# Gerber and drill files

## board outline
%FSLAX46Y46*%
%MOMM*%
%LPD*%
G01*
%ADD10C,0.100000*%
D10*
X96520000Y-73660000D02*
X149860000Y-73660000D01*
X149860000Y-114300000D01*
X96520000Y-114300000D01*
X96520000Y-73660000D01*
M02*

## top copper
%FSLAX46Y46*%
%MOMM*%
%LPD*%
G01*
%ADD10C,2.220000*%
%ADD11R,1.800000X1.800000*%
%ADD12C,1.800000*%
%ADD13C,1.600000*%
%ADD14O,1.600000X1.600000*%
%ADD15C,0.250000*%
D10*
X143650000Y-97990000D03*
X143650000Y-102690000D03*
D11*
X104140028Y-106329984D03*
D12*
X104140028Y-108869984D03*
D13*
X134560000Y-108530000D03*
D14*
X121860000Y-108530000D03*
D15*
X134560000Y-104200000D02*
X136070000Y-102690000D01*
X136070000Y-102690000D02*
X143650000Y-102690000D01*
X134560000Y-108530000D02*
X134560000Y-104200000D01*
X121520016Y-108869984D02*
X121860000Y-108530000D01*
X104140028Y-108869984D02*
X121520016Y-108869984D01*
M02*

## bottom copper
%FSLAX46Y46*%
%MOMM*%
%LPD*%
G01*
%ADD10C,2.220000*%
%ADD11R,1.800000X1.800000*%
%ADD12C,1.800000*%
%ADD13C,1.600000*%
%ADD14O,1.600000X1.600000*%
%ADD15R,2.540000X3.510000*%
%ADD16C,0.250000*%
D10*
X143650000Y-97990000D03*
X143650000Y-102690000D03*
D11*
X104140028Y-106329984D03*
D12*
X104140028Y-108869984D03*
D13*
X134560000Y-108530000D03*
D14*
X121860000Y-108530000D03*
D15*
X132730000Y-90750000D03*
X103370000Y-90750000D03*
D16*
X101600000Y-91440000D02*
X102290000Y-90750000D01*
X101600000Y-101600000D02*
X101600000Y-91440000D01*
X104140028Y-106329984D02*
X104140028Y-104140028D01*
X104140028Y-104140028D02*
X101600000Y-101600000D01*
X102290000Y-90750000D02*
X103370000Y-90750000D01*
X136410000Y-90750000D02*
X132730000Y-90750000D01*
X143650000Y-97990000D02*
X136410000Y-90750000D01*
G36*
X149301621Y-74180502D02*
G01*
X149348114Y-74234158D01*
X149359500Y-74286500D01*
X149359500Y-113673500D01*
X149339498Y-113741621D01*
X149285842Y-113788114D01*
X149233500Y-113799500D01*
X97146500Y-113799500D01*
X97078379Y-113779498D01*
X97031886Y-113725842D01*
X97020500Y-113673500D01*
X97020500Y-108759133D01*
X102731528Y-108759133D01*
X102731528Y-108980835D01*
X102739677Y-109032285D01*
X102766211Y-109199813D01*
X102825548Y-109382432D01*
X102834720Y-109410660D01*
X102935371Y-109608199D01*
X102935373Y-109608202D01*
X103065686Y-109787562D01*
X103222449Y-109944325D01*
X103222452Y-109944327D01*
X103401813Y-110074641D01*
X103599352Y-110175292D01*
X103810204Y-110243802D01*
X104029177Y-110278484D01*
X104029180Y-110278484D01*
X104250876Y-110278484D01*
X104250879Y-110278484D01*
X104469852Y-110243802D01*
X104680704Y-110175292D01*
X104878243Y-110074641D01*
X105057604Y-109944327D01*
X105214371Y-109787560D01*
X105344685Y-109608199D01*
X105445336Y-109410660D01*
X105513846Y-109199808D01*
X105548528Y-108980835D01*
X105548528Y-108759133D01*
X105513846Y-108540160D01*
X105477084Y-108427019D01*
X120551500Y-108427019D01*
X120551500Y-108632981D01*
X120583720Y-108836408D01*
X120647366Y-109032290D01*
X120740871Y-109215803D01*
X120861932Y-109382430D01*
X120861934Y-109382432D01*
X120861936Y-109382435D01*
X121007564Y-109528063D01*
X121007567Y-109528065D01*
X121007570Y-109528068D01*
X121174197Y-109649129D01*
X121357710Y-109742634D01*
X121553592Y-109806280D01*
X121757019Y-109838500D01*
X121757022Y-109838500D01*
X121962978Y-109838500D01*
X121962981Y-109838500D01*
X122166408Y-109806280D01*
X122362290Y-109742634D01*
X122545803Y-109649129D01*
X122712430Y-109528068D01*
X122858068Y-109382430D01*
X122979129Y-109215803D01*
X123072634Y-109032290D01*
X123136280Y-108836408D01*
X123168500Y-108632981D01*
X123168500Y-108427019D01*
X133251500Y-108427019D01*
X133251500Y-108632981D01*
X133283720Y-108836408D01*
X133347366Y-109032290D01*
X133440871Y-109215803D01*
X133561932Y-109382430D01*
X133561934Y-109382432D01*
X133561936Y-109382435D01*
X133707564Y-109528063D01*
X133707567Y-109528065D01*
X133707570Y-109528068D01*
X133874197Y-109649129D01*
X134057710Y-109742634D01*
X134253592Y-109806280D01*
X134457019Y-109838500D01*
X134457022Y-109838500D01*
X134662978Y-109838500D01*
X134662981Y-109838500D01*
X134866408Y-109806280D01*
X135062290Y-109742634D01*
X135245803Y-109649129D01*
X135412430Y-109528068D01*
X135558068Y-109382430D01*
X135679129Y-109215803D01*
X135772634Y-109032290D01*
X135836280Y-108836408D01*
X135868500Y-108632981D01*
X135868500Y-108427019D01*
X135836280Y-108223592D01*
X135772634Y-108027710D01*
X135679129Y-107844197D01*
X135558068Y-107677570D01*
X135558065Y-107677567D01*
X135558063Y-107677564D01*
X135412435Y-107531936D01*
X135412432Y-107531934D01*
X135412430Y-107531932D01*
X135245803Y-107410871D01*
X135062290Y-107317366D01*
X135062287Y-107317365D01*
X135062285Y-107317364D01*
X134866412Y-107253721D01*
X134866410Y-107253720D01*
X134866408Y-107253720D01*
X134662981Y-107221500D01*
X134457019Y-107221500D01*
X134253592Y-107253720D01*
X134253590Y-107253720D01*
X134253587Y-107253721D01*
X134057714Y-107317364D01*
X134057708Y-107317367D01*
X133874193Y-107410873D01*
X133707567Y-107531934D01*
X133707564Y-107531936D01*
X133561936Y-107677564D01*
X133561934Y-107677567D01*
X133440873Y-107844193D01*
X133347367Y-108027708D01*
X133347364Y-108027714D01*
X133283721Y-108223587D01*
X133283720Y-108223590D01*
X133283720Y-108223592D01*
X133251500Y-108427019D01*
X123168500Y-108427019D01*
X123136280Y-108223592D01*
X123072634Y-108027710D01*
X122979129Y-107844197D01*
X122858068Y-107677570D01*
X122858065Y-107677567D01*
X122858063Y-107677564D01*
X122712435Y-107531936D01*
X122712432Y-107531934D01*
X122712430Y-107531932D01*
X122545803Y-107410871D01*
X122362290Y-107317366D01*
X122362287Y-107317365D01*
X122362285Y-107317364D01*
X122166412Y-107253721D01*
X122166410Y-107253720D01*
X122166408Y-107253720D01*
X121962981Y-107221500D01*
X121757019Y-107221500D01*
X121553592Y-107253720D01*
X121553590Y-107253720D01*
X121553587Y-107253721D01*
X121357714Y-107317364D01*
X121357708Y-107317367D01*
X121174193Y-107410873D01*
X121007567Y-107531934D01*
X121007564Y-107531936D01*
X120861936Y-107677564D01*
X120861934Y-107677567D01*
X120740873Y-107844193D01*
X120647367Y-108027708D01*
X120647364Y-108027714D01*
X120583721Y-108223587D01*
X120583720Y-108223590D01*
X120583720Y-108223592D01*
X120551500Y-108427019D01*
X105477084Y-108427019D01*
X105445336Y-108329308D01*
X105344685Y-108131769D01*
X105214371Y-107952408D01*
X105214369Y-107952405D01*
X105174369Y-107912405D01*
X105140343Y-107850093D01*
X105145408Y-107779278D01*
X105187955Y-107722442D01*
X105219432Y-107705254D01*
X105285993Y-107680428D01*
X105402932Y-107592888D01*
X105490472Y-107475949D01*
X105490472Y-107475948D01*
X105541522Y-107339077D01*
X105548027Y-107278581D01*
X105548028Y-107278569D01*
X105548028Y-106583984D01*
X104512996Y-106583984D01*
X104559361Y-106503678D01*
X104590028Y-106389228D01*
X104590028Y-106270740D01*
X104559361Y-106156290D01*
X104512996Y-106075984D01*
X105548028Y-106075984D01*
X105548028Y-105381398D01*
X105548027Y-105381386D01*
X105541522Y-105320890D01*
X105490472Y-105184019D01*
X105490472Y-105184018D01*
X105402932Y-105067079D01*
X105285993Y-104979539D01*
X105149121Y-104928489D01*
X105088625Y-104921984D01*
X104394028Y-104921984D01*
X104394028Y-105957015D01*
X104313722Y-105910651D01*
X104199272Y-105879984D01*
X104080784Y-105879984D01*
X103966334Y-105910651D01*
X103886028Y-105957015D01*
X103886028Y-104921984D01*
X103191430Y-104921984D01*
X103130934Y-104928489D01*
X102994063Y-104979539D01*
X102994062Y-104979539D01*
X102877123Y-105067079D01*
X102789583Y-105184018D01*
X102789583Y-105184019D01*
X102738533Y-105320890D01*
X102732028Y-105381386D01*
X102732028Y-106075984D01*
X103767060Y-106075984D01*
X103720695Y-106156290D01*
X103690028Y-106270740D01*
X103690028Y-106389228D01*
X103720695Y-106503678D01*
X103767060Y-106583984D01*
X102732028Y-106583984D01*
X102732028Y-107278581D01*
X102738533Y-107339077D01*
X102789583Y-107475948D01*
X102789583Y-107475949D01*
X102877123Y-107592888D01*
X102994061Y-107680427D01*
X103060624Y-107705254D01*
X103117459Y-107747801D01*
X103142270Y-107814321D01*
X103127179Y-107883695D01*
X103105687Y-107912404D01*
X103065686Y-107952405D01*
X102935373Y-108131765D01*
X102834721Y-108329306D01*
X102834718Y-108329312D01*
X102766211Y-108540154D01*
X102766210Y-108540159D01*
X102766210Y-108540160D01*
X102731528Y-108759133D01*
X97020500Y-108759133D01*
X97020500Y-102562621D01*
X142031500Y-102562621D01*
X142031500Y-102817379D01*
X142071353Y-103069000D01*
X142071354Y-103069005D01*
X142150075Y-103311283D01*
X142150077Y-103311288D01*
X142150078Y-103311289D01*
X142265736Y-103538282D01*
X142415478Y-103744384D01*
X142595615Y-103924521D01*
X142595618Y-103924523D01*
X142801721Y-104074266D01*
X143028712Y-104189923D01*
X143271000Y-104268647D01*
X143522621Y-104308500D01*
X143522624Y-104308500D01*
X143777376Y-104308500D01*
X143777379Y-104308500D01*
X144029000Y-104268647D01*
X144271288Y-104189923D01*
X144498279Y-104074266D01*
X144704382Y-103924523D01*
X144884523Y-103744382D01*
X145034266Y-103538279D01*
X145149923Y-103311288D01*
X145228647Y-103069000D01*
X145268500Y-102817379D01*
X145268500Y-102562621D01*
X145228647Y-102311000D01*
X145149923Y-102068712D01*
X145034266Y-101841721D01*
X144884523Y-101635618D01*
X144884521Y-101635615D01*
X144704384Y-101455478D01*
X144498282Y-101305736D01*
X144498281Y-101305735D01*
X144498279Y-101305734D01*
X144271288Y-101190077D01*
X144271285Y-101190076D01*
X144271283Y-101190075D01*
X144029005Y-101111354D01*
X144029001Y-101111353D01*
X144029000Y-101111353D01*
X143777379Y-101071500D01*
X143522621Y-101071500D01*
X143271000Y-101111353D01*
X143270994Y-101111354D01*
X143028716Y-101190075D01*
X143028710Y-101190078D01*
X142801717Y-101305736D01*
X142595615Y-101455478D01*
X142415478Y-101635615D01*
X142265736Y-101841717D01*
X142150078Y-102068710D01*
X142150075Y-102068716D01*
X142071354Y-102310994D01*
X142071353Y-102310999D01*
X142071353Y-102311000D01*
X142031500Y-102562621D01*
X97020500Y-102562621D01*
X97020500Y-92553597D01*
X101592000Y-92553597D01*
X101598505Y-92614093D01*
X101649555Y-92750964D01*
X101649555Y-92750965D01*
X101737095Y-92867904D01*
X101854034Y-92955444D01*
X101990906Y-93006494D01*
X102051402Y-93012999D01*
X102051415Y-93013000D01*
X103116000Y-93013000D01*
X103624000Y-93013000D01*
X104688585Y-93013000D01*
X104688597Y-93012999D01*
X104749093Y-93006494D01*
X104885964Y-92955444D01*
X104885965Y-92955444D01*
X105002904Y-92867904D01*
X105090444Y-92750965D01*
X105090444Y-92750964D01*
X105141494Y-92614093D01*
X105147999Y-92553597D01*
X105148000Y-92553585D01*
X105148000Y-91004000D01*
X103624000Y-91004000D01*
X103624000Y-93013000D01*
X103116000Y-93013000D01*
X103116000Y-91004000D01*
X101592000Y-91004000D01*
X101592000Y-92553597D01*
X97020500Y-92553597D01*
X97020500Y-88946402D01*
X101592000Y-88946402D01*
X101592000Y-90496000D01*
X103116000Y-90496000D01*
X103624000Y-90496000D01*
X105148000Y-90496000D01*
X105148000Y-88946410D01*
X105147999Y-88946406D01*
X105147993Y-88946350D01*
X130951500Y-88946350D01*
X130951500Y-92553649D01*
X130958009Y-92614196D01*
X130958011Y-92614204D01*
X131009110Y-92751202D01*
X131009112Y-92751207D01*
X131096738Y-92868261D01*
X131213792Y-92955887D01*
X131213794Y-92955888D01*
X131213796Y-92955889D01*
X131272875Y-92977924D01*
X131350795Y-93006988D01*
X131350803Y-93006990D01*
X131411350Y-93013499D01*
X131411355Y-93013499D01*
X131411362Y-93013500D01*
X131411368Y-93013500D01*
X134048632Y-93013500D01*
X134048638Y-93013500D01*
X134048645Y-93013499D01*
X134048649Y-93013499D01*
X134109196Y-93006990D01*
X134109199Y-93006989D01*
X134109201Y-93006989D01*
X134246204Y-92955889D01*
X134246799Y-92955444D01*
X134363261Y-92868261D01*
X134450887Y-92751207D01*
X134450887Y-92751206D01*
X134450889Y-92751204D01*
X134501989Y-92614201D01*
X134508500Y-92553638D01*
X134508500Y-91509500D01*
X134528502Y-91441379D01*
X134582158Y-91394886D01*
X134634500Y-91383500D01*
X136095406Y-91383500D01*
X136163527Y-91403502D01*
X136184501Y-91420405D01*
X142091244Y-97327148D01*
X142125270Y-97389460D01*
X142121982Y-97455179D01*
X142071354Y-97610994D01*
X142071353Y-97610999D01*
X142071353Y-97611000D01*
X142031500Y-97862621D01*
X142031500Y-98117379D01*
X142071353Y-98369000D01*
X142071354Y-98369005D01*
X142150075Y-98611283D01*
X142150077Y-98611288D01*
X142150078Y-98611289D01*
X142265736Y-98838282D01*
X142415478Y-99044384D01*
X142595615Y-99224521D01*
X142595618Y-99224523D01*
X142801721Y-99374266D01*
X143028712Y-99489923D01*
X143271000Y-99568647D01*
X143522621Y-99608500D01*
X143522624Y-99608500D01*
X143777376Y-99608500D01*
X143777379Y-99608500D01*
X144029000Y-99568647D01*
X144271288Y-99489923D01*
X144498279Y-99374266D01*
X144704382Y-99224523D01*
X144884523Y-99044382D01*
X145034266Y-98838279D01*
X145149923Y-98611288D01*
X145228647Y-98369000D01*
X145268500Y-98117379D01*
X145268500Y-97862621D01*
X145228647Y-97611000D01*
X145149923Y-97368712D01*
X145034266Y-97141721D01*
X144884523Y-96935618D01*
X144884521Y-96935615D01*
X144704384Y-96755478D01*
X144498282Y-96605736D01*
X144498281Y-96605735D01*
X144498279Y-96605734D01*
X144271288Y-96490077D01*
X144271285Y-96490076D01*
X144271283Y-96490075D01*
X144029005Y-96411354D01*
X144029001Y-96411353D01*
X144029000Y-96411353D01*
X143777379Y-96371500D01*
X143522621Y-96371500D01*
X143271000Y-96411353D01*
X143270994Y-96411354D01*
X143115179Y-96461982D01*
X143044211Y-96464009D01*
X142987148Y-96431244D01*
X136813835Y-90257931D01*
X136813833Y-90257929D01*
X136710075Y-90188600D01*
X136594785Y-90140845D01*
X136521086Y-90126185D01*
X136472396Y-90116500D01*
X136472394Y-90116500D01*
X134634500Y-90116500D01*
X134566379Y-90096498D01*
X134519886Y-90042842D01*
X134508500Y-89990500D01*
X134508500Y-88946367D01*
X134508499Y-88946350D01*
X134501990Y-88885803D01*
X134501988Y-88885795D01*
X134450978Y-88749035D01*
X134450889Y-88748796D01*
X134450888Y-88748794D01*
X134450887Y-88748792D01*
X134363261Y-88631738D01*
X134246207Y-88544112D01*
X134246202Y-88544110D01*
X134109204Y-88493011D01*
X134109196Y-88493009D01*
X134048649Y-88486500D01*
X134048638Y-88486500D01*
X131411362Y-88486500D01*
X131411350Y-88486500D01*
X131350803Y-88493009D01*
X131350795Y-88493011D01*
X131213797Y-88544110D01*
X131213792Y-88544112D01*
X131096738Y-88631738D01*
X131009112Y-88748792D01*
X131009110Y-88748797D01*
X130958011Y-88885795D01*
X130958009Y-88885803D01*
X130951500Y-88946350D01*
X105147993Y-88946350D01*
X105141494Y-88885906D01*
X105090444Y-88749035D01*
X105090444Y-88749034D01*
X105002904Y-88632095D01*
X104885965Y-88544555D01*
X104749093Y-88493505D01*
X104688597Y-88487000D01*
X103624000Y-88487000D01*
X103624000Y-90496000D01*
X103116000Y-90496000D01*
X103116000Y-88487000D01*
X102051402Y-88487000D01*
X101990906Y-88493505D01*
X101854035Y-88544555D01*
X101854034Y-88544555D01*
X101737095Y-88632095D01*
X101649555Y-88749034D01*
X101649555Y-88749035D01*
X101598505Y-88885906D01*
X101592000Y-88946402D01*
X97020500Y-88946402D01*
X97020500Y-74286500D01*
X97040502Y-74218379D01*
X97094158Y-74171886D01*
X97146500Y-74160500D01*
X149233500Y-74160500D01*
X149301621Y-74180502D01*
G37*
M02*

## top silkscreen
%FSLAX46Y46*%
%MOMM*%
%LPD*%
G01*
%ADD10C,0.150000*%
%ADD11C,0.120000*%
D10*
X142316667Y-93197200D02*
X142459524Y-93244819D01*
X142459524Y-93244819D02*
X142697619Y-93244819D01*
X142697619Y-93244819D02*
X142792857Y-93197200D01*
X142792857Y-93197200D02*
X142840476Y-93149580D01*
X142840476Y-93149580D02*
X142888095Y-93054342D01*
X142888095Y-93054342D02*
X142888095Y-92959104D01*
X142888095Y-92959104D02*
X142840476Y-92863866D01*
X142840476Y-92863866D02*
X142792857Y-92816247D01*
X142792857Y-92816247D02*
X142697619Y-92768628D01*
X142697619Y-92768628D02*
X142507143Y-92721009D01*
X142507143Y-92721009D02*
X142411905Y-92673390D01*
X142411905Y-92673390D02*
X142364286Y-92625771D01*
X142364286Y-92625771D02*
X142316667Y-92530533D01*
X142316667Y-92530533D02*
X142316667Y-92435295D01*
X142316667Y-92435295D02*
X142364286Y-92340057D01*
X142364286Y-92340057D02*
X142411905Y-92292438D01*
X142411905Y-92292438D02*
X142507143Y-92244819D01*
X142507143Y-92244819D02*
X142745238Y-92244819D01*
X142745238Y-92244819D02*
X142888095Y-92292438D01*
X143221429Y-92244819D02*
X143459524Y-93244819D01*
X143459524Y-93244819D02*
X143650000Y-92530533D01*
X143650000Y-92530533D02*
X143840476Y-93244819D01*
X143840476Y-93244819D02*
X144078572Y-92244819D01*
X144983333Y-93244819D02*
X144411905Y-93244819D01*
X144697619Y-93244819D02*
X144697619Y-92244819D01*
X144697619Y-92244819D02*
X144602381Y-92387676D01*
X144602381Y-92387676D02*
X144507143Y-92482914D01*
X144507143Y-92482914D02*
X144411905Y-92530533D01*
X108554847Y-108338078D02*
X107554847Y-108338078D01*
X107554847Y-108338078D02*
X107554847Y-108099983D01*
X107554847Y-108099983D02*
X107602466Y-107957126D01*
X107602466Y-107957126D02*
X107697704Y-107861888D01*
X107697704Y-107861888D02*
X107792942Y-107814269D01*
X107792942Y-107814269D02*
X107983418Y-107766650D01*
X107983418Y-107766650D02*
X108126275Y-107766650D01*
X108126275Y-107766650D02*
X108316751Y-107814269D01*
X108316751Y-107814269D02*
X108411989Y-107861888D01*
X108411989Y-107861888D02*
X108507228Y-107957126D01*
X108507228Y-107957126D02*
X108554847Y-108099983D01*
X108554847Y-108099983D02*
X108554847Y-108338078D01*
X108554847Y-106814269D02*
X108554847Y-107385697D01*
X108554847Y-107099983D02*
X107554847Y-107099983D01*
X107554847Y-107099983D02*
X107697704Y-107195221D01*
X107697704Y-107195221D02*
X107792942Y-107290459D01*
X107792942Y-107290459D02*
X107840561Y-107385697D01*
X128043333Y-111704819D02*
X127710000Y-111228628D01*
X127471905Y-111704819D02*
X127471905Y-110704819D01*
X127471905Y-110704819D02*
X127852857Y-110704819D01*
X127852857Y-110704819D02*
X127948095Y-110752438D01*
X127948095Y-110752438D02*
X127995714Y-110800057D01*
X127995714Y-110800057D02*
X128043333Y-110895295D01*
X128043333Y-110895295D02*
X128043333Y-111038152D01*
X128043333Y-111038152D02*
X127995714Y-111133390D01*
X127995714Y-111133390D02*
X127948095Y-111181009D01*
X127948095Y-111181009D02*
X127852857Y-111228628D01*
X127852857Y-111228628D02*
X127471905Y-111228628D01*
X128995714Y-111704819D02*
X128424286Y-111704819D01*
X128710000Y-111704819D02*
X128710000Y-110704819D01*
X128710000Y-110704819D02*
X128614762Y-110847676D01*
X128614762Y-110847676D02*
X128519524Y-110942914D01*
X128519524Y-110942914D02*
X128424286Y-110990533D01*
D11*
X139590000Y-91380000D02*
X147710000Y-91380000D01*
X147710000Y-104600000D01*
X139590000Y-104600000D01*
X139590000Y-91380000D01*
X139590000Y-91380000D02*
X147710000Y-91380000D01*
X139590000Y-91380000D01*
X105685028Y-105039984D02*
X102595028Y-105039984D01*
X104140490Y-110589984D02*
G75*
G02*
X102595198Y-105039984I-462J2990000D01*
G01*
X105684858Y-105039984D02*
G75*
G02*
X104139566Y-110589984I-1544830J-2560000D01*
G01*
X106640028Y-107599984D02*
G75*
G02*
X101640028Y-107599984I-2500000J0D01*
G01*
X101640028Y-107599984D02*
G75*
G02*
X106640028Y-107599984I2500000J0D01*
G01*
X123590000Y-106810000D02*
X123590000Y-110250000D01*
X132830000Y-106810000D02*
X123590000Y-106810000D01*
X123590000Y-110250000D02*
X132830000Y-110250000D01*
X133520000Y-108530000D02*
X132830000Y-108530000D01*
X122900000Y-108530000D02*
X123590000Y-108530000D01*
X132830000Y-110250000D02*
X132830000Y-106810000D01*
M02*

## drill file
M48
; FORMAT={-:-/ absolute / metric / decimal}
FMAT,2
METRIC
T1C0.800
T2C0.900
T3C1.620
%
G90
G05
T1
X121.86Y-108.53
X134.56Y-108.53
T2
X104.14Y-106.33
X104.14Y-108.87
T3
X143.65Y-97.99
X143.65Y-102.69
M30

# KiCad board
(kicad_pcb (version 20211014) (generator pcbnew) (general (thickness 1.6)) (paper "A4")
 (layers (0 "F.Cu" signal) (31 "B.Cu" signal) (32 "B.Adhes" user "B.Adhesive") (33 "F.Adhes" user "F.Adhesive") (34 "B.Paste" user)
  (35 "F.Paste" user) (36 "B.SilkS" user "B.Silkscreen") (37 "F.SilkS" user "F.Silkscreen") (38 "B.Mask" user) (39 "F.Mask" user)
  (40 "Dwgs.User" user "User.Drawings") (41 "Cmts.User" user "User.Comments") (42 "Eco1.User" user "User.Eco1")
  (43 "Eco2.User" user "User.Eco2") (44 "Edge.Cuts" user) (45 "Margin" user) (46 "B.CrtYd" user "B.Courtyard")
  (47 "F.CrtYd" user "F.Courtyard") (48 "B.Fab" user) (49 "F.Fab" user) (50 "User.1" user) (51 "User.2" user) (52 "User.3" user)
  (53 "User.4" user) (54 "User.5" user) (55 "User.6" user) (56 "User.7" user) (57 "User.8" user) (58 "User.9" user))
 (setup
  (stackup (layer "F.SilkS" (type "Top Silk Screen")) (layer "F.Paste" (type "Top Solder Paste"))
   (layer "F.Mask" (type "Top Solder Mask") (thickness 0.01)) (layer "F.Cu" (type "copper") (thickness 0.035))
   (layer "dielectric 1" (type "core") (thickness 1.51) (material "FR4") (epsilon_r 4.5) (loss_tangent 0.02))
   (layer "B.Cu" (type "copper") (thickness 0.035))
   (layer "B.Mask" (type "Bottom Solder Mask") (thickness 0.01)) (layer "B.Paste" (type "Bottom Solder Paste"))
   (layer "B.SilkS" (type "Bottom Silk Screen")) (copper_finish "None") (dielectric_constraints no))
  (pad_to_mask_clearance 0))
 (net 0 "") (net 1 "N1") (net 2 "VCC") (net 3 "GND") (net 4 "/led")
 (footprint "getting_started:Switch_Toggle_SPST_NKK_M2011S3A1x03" (layer "F.Cu") (at 143.65 93.29)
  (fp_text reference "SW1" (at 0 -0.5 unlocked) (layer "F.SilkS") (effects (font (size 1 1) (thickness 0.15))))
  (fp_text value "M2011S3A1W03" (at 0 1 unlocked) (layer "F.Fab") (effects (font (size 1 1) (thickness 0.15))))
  (fp_rect (start 4.06 11.31) (end -4.06 -1.91) (layer "F.SilkS") (width 0.12) (fill none))
  (fp_rect (start -4.06 -1.91) (end 4.06 -1.91) (layer "F.SilkS") (width 0.12) (fill none))
  (pad "2" thru_hole circle (at 0 4.7) (size 2.22 2.22) (drill 1.62) (layers *.Cu *.Mask) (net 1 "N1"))
  (pad "3" thru_hole circle (at 0 9.4) (size 2.22 2.22) (drill 1.62) (layers *.Cu *.Mask) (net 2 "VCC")))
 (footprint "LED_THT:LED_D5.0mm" (layer "F.Cu") (at 104.140028 106.329984 -90)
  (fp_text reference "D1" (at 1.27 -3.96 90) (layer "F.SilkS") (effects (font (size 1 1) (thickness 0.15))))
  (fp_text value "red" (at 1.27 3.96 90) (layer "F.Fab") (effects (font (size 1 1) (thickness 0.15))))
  (fp_line (start -1.29 -1.545) (end -1.29 1.545) (layer "F.SilkS") (width 0.12))
  (fp_arc (start 4.26 -0.000462) (mid 2.072002 2.880433) (end -1.29 1.54483) (layer "F.SilkS") (width 0.12))
  (fp_arc (start -1.29 -1.54483) (mid 2.072002 -2.880433) (end 4.26 0.000462) (layer "F.SilkS") (width 0.12))
  (fp_circle (center 1.27 0) (end 3.77 0) (layer "F.SilkS") (width 0.12) (fill none))
  (pad "1" thru_hole rect (at 0 0 270) (size 1.8 1.8) (drill 0.9) (layers *.Cu *.Mask) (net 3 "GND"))
  (pad "2" thru_hole circle (at 2.54 0 270) (size 1.8 1.8) (drill 0.9) (layers *.Cu *.Mask) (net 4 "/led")))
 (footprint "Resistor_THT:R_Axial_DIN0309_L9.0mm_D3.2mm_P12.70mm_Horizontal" (layer "F.Cu") (at 134.56 108.53 180)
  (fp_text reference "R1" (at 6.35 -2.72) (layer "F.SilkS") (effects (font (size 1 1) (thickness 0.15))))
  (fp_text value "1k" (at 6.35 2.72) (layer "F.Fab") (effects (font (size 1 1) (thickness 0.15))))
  (fp_line (start 10.97 1.72) (end 10.97 -1.72) (layer "F.SilkS") (width 0.12))
  (fp_line (start 1.73 1.72) (end 10.97 1.72) (layer "F.SilkS") (width 0.12))
  (fp_line (start 10.97 -1.72) (end 1.73 -1.72) (layer "F.SilkS") (width 0.12))
  (fp_line (start 1.04 0) (end 1.73 0) (layer "F.SilkS") (width 0.12))
  (fp_line (start 11.66 0) (end 10.97 0) (layer "F.SilkS") (width 0.12))
  (fp_line (start 1.73 -1.72) (end 1.73 1.72) (layer "F.SilkS") (width 0.12))
  (pad "1" thru_hole circle (at 0 0 180) (size 1.6 1.6) (drill 0.8) (layers *.Cu *.Mask) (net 2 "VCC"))
  (pad "2" thru_hole oval (at 12.7 0 180) (size 1.6 1.6) (drill 0.8) (layers *.Cu *.Mask) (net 4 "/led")))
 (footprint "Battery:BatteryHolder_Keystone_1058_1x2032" (layer "B.Cu") (at 118.05 90.75 180)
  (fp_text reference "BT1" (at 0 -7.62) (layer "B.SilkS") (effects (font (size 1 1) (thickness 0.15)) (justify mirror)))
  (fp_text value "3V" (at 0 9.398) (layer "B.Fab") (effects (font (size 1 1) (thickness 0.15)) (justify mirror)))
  (pad "1" smd rect (at -14.68 0 180) (size 2.54 3.51) (layers "B.Cu" "B.Paste" "B.Mask") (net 1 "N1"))
  (pad "2" smd rect (at 14.68 0 180) (size 2.54 3.51) (layers "B.Cu" "B.Paste" "B.Mask") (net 3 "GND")))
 (gr_rect (start 96.52 73.66) (end 149.86 114.3) (layer "Edge.Cuts") (width 0.1) (fill none))
 (segment (start 134.56 104.2) (end 136.07 102.69) (width 0.25) (layer "F.Cu") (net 2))
 (segment (start 136.07 102.69) (end 143.65 102.69) (width 0.25) (layer "F.Cu") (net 2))
 (segment (start 134.56 108.53) (end 134.56 104.2) (width 0.25) (layer "F.Cu") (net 2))
 (segment (start 101.6 91.44) (end 102.29 90.75) (width 0.25) (layer "B.Cu") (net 3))
 (segment (start 101.6 101.6) (end 101.6 91.44) (width 0.25) (layer "B.Cu") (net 3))
 (segment (start 104.140028 106.329984) (end 104.140028 104.140028) (width 0.25) (layer "B.Cu") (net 3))
 (segment (start 104.140028 104.140028) (end 101.6 101.6) (width 0.25) (layer "B.Cu") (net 3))
 (segment (start 102.29 90.75) (end 103.37 90.75) (width 0.25) (layer "B.Cu") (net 3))
 (segment (start 121.520016 108.869984) (end 121.86 108.53) (width 0.25) (layer "F.Cu") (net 4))
 (segment (start 104.140028 108.869984) (end 121.520016 108.869984) (width 0.25) (layer "F.Cu") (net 4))
 (segment (start 136.41 90.75) (end 132.73 90.75) (width 0.25) (layer "B.Cu") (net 1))
 (segment (start 143.65 97.99) (end 136.41 90.75) (width 0.25) (layer "B.Cu") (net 1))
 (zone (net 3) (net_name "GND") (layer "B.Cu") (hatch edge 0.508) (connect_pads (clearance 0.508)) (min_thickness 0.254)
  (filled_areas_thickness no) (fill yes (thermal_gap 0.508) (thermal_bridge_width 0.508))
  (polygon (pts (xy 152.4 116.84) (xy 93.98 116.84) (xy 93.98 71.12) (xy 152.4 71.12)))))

